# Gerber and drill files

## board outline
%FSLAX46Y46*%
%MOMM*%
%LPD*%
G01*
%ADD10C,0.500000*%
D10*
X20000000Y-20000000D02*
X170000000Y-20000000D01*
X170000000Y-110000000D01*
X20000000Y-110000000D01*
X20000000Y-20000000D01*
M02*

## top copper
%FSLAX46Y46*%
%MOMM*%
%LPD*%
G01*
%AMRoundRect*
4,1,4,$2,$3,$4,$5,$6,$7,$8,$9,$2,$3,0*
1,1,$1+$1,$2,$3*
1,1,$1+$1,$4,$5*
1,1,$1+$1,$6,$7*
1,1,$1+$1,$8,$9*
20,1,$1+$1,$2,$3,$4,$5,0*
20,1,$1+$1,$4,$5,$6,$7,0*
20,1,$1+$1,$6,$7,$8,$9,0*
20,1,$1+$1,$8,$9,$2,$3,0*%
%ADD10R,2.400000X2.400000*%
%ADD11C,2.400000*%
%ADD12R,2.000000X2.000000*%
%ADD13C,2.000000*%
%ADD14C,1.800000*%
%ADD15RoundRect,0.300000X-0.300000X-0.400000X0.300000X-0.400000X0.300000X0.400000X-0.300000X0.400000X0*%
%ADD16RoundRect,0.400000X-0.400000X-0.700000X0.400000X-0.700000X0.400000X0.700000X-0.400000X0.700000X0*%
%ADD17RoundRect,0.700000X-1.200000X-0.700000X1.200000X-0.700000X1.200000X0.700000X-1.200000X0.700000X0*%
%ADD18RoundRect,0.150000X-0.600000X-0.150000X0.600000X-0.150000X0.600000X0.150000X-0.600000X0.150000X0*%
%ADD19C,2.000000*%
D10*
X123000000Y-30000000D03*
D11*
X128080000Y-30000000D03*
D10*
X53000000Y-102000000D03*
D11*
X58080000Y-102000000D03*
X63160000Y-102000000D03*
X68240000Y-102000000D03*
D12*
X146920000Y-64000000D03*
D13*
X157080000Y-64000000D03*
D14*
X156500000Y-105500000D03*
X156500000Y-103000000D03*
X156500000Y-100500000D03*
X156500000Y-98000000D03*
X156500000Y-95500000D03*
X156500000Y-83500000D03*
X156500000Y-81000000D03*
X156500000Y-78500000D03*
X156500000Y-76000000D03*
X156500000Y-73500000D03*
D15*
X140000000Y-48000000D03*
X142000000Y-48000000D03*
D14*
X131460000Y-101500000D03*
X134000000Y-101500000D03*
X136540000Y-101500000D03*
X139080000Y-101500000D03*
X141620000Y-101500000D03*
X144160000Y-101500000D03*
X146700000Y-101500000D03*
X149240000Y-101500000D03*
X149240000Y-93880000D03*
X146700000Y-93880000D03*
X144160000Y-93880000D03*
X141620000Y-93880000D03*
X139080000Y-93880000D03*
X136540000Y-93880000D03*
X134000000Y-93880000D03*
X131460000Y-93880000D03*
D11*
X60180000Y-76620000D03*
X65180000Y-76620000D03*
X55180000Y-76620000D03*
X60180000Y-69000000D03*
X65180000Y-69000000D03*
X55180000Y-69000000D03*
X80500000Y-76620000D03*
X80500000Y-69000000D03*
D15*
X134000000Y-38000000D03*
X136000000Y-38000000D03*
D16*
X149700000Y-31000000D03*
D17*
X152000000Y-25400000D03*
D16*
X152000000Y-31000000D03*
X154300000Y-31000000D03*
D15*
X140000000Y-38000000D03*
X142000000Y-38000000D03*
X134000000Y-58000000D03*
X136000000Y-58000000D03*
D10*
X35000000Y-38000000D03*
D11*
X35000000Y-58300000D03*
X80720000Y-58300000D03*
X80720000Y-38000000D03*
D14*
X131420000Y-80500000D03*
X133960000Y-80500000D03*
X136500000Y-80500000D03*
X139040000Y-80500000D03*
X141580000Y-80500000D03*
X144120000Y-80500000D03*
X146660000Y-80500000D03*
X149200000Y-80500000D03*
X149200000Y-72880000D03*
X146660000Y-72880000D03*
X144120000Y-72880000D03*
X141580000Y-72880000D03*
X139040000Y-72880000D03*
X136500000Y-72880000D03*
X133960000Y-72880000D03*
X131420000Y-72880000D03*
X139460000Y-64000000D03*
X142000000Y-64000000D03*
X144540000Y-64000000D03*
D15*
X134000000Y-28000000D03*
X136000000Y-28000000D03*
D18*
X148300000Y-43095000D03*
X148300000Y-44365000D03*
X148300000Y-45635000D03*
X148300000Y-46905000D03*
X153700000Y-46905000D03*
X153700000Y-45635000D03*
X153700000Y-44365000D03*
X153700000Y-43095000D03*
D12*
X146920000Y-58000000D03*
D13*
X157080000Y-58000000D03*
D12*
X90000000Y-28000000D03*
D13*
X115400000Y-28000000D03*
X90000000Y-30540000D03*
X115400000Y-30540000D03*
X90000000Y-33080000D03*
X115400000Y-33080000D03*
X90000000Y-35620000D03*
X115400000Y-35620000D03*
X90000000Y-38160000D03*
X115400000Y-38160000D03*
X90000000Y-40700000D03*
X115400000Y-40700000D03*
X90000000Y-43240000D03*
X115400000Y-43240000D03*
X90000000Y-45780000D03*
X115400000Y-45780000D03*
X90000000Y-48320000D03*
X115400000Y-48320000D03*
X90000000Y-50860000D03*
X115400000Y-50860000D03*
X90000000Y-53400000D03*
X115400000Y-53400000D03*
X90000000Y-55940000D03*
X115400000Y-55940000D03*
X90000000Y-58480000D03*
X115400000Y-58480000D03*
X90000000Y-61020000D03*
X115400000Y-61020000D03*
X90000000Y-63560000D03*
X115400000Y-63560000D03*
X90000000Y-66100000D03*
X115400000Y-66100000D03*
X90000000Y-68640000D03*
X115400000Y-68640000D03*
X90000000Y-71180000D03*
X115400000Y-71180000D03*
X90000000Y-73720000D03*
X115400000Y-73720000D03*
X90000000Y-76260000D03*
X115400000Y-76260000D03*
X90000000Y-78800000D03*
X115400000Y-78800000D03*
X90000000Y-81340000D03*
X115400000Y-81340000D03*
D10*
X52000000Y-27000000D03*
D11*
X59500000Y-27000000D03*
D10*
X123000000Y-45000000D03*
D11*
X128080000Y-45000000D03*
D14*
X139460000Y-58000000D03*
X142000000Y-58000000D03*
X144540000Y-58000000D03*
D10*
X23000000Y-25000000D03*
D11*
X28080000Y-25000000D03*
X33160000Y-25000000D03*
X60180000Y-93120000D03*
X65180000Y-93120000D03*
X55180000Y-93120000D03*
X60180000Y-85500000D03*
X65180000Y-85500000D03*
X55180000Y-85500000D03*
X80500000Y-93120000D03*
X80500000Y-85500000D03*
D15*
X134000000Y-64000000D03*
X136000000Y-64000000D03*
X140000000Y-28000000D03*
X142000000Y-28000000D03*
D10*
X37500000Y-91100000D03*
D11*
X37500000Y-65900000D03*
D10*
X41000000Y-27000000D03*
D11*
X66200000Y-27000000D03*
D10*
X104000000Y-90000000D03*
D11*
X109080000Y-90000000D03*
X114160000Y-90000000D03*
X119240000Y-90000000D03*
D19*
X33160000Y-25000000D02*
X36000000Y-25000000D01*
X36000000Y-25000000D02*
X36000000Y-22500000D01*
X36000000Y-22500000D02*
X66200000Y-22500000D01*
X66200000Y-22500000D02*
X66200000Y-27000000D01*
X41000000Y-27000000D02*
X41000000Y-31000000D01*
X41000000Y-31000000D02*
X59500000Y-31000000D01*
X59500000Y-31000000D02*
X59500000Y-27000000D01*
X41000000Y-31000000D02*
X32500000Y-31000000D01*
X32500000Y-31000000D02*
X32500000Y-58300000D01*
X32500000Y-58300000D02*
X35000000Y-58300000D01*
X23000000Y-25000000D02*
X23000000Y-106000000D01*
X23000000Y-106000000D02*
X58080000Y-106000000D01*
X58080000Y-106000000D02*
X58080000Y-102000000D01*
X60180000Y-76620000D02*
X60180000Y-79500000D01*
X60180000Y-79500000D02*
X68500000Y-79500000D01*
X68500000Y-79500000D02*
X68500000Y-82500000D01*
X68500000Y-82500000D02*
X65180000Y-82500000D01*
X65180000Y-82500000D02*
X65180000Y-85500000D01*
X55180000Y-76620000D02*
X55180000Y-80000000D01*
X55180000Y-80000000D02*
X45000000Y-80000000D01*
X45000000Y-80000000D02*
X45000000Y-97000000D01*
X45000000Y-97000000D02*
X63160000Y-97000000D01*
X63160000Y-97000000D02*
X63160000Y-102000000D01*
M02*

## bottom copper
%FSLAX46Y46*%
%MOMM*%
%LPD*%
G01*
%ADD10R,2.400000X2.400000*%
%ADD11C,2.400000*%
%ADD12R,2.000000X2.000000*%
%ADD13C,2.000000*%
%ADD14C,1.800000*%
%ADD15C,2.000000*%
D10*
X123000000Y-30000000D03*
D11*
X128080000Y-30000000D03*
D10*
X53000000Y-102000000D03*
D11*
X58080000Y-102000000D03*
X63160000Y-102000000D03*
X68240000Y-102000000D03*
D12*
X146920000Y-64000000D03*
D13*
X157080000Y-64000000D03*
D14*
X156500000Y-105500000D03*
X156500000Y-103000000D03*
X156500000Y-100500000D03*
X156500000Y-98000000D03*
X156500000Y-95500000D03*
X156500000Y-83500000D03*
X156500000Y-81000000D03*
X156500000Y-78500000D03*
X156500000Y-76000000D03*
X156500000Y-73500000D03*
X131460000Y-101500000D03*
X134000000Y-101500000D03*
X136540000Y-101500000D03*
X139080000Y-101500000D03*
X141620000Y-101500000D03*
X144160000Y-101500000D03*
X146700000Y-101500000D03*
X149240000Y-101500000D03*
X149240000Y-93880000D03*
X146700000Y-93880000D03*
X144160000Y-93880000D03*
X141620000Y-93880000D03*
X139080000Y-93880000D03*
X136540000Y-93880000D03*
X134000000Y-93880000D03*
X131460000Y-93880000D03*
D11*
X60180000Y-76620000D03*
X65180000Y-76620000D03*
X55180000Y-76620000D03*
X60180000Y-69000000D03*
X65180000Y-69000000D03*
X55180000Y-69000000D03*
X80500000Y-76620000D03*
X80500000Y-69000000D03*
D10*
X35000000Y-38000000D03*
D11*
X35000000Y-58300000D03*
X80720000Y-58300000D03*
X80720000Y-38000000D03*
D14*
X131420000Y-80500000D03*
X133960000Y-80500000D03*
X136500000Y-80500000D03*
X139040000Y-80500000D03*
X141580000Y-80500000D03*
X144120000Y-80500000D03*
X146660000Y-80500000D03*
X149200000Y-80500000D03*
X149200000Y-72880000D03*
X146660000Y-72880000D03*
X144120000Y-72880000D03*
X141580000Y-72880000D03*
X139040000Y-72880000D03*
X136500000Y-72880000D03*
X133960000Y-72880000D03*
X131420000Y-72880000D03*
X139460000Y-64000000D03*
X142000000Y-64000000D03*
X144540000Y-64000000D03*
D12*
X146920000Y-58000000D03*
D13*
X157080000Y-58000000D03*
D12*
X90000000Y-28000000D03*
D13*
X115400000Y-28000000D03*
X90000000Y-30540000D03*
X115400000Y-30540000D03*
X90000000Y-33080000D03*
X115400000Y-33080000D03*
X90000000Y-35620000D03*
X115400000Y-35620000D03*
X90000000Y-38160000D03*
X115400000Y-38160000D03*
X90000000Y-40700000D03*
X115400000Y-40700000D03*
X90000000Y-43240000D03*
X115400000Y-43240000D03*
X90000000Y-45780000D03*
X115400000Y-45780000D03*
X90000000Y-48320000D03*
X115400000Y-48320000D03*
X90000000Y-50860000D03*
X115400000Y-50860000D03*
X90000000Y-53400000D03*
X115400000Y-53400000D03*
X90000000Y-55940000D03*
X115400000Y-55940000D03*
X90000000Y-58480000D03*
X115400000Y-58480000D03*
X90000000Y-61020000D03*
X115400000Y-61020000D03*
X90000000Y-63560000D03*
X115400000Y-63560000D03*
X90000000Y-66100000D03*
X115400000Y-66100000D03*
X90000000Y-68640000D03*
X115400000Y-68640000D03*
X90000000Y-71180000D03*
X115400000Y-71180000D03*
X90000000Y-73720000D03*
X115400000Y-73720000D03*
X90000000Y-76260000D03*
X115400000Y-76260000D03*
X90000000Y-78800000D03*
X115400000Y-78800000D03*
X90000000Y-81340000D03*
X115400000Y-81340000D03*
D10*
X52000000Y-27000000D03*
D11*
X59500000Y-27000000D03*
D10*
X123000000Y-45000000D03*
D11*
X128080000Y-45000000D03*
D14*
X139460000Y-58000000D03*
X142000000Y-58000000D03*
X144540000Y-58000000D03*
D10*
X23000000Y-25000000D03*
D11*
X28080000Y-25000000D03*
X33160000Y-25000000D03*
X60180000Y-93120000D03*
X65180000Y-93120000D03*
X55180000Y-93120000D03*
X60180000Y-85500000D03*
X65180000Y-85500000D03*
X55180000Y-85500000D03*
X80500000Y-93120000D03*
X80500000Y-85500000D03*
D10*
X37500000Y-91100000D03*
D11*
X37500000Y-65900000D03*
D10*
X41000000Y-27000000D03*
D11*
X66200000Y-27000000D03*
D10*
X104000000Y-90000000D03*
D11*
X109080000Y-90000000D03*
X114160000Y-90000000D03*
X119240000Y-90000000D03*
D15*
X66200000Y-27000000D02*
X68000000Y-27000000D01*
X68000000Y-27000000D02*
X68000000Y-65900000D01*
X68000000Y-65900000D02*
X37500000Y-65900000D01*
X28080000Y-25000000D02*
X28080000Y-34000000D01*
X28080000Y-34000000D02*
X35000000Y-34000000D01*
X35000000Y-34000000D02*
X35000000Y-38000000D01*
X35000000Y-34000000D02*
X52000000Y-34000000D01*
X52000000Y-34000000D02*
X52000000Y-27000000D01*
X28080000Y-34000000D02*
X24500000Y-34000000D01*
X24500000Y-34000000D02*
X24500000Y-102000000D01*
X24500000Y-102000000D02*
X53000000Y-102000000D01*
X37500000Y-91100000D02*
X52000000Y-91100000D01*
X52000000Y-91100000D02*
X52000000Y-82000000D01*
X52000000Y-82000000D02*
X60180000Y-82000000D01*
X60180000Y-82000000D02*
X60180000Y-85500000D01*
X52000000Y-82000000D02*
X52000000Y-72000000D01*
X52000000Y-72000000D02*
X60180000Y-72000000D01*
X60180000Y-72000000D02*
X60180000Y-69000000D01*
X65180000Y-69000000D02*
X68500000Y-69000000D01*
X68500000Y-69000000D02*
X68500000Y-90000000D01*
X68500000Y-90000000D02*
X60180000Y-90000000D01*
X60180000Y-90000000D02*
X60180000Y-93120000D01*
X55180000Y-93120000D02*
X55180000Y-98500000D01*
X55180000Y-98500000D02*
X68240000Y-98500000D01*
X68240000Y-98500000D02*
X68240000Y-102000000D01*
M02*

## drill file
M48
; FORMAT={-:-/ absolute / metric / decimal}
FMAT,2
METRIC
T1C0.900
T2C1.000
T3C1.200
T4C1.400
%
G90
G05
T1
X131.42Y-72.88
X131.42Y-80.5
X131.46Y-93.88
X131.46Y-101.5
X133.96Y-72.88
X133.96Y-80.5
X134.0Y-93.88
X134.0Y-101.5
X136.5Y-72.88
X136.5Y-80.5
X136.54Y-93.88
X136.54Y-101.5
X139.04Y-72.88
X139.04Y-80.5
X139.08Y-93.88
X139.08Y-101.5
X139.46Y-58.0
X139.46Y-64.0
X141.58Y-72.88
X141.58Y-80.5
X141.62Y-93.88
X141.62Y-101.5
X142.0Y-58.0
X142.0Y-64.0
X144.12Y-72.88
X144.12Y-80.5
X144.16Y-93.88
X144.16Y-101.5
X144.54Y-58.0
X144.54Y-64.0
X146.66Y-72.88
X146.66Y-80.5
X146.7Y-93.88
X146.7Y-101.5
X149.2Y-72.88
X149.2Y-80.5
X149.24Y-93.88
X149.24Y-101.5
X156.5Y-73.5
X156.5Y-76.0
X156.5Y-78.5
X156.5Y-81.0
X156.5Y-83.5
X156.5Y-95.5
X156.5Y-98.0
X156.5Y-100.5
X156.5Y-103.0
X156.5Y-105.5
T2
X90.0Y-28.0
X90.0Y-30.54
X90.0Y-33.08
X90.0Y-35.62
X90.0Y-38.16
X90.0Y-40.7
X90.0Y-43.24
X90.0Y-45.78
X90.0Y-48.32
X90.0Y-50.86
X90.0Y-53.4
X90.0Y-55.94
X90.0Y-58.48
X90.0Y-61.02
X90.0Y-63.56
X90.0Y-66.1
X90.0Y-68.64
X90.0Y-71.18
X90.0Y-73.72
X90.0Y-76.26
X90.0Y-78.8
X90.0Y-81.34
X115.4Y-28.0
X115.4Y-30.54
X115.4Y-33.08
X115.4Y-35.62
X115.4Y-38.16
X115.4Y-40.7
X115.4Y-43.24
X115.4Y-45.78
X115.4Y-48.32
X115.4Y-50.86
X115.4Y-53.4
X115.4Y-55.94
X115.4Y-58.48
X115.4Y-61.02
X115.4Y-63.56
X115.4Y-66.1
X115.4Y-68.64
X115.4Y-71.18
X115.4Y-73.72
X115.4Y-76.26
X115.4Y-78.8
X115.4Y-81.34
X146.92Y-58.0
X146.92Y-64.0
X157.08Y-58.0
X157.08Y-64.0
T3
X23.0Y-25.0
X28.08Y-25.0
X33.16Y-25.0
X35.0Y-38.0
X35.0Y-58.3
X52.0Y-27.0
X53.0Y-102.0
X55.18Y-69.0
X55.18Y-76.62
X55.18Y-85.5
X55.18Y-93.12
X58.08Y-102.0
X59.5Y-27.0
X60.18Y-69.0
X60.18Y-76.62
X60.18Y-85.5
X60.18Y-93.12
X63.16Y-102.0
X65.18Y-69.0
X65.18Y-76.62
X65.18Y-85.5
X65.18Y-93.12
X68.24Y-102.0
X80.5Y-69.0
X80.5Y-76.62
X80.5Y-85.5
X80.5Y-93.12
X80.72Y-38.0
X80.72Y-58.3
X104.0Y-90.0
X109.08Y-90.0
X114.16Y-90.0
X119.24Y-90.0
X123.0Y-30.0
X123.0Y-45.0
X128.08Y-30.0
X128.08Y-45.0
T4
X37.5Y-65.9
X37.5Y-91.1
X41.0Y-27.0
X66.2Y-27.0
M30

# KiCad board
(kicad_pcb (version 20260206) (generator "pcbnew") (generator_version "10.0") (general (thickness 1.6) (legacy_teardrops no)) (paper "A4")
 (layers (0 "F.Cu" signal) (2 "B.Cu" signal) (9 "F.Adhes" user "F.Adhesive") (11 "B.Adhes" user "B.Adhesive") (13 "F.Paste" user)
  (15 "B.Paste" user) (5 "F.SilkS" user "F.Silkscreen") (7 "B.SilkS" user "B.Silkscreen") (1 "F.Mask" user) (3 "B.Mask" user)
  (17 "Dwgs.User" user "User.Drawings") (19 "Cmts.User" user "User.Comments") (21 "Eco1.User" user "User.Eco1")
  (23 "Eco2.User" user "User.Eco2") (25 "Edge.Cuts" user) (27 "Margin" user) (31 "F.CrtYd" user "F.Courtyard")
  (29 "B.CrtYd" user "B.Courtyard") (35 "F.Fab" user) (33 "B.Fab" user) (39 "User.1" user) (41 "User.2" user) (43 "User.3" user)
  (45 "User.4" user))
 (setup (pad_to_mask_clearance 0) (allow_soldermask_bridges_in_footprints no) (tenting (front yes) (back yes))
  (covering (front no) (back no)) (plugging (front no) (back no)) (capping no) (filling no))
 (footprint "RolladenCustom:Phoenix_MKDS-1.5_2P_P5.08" (layer "F.Cu") (at 123 30)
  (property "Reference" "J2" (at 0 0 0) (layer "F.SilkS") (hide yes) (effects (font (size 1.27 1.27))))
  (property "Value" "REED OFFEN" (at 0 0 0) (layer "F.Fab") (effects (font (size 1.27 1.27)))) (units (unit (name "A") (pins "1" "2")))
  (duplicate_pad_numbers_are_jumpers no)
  (pad "1" thru_hole rect (at 0 0) (size 2.4 2.4) (drill 1.2) (layers "*.Cu" "*.Mask") (remove_unused_layers no) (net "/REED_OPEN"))
  (pad "2" thru_hole circle (at 5.08 0) (size 2.4 2.4) (drill 1.2) (layers "*.Cu" "*.Mask") (remove_unused_layers no) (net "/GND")))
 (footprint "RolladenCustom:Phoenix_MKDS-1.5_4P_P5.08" (layer "F.Cu") (at 53 102)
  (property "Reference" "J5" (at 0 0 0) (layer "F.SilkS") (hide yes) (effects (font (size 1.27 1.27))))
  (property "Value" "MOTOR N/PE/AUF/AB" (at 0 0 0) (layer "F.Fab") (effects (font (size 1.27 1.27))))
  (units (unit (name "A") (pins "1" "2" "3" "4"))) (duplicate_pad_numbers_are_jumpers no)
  (pad "1" thru_hole rect (at 0 0) (size 2.4 2.4) (drill 1.2) (layers "*.Cu" "*.Mask") (remove_unused_layers no) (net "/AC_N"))
  (pad "2" thru_hole circle (at 5.08 0) (size 2.4 2.4) (drill 1.2) (layers "*.Cu" "*.Mask") (remove_unused_layers no) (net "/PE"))
  (pad "3" thru_hole circle (at 10.16 0) (size 2.4 2.4) (drill 1.2) (layers "*.Cu" "*.Mask") (remove_unused_layers no) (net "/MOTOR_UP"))
  (pad "4" thru_hole circle (at 15.24 0) (size 2.4 2.4) (drill 1.2) (layers "*.Cu" "*.Mask") (remove_unused_layers no) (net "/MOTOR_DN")))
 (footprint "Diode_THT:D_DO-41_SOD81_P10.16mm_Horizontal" (layer "F.Cu") (at 152 64)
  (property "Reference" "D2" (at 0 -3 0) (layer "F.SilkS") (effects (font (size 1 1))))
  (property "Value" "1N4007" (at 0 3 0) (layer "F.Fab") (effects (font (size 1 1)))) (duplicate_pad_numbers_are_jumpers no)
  (pad "1" thru_hole rect (at -5.08 0) (size 2 2) (drill 1) (layers "*.Cu" "*.Mask") (remove_unused_layers no) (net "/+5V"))
  (pad "2" thru_hole circle (at 5.08 0) (size 2 2) (drill 1) (layers "*.Cu" "*.Mask") (remove_unused_layers no) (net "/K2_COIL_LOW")))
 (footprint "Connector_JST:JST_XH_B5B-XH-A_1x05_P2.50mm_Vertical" (layer "F.Cu") (at 156.5 105.5 90)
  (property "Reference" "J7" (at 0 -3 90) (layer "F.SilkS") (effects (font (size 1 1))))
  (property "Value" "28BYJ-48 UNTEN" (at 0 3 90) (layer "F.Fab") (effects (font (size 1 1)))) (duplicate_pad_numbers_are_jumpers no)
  (pad "1" thru_hole circle (at 0 0 90) (size 1.8 1.8) (drill 0.9) (layers "*.Cu" "*.Mask") (remove_unused_layers no) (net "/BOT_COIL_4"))
  (pad "2" thru_hole circle (at 2.5 0 90) (size 1.8 1.8) (drill 0.9) (layers "*.Cu" "*.Mask") (remove_unused_layers no) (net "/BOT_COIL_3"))
  (pad "3" thru_hole circle (at 5 0 90) (size 1.8 1.8) (drill 0.9) (layers "*.Cu" "*.Mask") (remove_unused_layers no) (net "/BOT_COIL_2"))
  (pad "4" thru_hole circle (at 7.5 0 90) (size 1.8 1.8) (drill 0.9) (layers "*.Cu" "*.Mask") (remove_unused_layers no) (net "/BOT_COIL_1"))
  (pad "5" thru_hole circle (at 10 0 90) (size 1.8 1.8) (drill 0.9) (layers "*.Cu" "*.Mask") (remove_unused_layers no) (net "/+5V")))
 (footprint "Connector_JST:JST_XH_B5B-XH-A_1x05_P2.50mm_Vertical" (layer "F.Cu") (at 156.5 83.5 90)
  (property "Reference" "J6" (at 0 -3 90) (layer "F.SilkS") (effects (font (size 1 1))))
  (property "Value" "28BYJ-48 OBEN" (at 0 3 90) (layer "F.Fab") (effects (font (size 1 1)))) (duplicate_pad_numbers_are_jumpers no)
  (pad "1" thru_hole circle (at 0 0 90) (size 1.8 1.8) (drill 0.9) (layers "*.Cu" "*.Mask") (remove_unused_layers no) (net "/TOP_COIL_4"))
  (pad "2" thru_hole circle (at 2.5 0 90) (size 1.8 1.8) (drill 0.9) (layers "*.Cu" "*.Mask") (remove_unused_layers no) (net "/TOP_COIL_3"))
  (pad "3" thru_hole circle (at 5 0 90) (size 1.8 1.8) (drill 0.9) (layers "*.Cu" "*.Mask") (remove_unused_layers no) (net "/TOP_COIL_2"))
  (pad "4" thru_hole circle (at 7.5 0 90) (size 1.8 1.8) (drill 0.9) (layers "*.Cu" "*.Mask") (remove_unused_layers no) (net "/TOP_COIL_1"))
  (pad "5" thru_hole circle (at 10 0 90) (size 1.8 1.8) (drill 0.9) (layers "*.Cu" "*.Mask") (remove_unused_layers no) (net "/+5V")))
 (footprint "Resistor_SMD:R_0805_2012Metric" (layer "F.Cu") (at 141 48)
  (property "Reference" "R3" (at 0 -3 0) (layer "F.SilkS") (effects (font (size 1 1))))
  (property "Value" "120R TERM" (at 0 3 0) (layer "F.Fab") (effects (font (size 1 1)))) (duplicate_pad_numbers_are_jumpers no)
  (pad "1" smd roundrect (at -1 0) (size 1.2 1.4) (layers "F.Cu" "F.Mask" "F.Paste") (roundrect_rratio 0.25) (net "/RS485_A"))
  (pad "2" smd roundrect (at 1 0) (size 1.2 1.4) (layers "F.Cu" "F.Mask" "F.Paste") (roundrect_rratio 0.25) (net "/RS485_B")))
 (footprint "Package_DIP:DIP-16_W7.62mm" (layer "F.Cu") (at 131.46 101.5 90)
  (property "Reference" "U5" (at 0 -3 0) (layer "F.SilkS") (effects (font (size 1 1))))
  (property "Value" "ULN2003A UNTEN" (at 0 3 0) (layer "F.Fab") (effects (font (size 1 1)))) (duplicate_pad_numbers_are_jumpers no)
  (pad "1" thru_hole circle (at 0 0) (size 1.8 1.8) (drill 0.9) (layers "*.Cu" "*.Mask") (remove_unused_layers no) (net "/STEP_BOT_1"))
  (pad "2" thru_hole circle (at 0 2.54) (size 1.8 1.8) (drill 0.9) (layers "*.Cu" "*.Mask") (remove_unused_layers no) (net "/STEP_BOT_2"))
  (pad "3" thru_hole circle (at 0 5.08) (size 1.8 1.8) (drill 0.9) (layers "*.Cu" "*.Mask") (remove_unused_layers no) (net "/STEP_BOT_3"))
  (pad "4" thru_hole circle (at 0 7.62) (size 1.8 1.8) (drill 0.9) (layers "*.Cu" "*.Mask") (remove_unused_layers no) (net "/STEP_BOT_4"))
  (pad "5" thru_hole circle (at 0 10.16) (size 1.8 1.8) (drill 0.9) (layers "*.Cu" "*.Mask") (remove_unused_layers no))
  (pad "6" thru_hole circle (at 0 12.7) (size 1.8 1.8) (drill 0.9) (layers "*.Cu" "*.Mask") (remove_unused_layers no))
  (pad "7" thru_hole circle (at 0 15.24) (size 1.8 1.8) (drill 0.9) (layers "*.Cu" "*.Mask") (remove_unused_layers no))
  (pad "8" thru_hole circle (at 0 17.78) (size 1.8 1.8) (drill 0.9) (layers "*.Cu" "*.Mask") (remove_unused_layers no) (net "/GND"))
  (pad "9" thru_hole circle (at 7.62 17.78) (size 1.8 1.8) (drill 0.9) (layers "*.Cu" "*.Mask") (remove_unused_layers no) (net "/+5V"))
  (pad "10" thru_hole circle (at 7.62 15.24) (size 1.8 1.8) (drill 0.9) (layers "*.Cu" "*.Mask") (remove_unused_layers no))
  (pad "11" thru_hole circle (at 7.62 12.7) (size 1.8 1.8) (drill 0.9) (layers "*.Cu" "*.Mask") (remove_unused_layers no))
  (pad "12" thru_hole circle (at 7.62 10.16) (size 1.8 1.8) (drill 0.9) (layers "*.Cu" "*.Mask") (remove_unused_layers no))
  (pad "13" thru_hole circle (at 7.62 7.62) (size 1.8 1.8) (drill 0.9) (layers "*.Cu" "*.Mask") (remove_unused_layers no)
   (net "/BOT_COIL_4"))
  (pad "14" thru_hole circle (at 7.62 5.08) (size 1.8 1.8) (drill 0.9) (layers "*.Cu" "*.Mask") (remove_unused_layers no)
   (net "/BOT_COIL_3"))
  (pad "15" thru_hole circle (at 7.62 2.54) (size 1.8 1.8) (drill 0.9) (layers "*.Cu" "*.Mask") (remove_unused_layers no)
   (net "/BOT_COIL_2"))
  (pad "16" thru_hole circle (at 7.62 0) (size 1.8 1.8) (drill 0.9) (layers "*.Cu" "*.Mask") (remove_unused_layers no) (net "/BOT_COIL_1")))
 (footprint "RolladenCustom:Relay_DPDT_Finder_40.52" (layer "F.Cu") (at 80.5 76.62 180)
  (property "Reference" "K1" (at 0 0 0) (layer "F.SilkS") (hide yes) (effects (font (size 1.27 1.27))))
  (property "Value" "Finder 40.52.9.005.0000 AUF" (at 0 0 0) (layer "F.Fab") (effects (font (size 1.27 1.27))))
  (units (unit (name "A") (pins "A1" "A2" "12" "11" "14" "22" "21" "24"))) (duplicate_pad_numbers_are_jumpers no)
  (pad "11" thru_hole circle (at 20.32 0) (size 2.4 2.4) (drill 1.2) (layers "*.Cu" "*.Mask") (remove_unused_layers no) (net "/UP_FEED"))
  (pad "12" thru_hole circle (at 15.32 0) (size 2.4 2.4) (drill 1.2) (layers "*.Cu" "*.Mask") (remove_unused_layers no)
   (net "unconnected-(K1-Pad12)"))
  (pad "14" thru_hole circle (at 25.32 0) (size 2.4 2.4) (drill 1.2) (layers "*.Cu" "*.Mask") (remove_unused_layers no) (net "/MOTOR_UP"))
  (pad "21" thru_hole circle (at 20.32 7.62) (size 2.4 2.4) (drill 1.2) (layers "*.Cu" "*.Mask") (remove_unused_layers no) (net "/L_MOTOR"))
  (pad "22" thru_hole circle (at 15.32 7.62) (size 2.4 2.4) (drill 1.2) (layers "*.Cu" "*.Mask") (remove_unused_layers no) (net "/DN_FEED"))
  (pad "24" thru_hole circle (at 25.32 7.62) (size 2.4 2.4) (drill 1.2) (layers "*.Cu" "*.Mask") (remove_unused_layers no)
   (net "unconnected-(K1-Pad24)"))
  (pad "A1" thru_hole circle (at 0 0) (size 2.4 2.4) (drill 1.2) (layers "*.Cu" "*.Mask") (remove_unused_layers no) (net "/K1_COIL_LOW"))
  (pad "A2" thru_hole circle (at 0 7.62) (size 2.4 2.4) (drill 1.2) (layers "*.Cu" "*.Mask") (remove_unused_layers no) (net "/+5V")))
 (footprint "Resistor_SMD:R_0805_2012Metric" (layer "F.Cu") (at 135 38)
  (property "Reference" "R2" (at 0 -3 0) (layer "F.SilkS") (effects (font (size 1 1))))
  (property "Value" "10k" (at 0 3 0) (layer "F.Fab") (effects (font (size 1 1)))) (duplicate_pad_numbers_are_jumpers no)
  (pad "1" smd roundrect (at -1 0) (size 1.2 1.4) (layers "F.Cu" "F.Mask" "F.Paste") (roundrect_rratio 0.25) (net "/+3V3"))
  (pad "2" smd roundrect (at 1 0) (size 1.2 1.4) (layers "F.Cu" "F.Mask" "F.Paste") (roundrect_rratio 0.25) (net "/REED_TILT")))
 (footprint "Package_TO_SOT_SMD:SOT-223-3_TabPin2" (layer "F.Cu") (at 152 28)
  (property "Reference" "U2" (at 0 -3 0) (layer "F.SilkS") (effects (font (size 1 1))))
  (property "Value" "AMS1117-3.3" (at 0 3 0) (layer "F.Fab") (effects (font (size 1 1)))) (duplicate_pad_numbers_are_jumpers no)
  (pad "1" smd roundrect (at -2.3 3) (size 1.6 2.2) (layers "F.Cu" "F.Mask" "F.Paste") (roundrect_rratio 0.25) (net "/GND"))
  (pad "2" smd roundrect (at 0 -2.6) (size 3.8 2.8) (layers "F.Cu" "F.Mask" "F.Paste") (roundrect_rratio 0.25) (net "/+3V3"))
  (pad "2" smd roundrect (at 0 3) (size 1.6 2.2) (layers "F.Cu" "F.Mask" "F.Paste") (roundrect_rratio 0.25) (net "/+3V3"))
  (pad "3" smd roundrect (at 2.3 3) (size 1.6 2.2) (layers "F.Cu" "F.Mask" "F.Paste") (roundrect_rratio 0.25) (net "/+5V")))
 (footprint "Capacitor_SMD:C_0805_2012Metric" (layer "F.Cu") (at 141 38)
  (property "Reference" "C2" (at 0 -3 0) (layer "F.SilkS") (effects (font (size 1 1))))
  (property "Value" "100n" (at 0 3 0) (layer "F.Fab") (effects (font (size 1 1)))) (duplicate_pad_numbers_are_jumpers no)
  (pad "1" smd roundrect (at -1 0) (size 1.2 1.4) (layers "F.Cu" "F.Mask" "F.Paste") (roundrect_rratio 0.25) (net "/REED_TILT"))
  (pad "2" smd roundrect (at 1 0) (size 1.2 1.4) (layers "F.Cu" "F.Mask" "F.Paste") (roundrect_rratio 0.25) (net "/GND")))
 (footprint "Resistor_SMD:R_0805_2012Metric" (layer "F.Cu") (at 135 58)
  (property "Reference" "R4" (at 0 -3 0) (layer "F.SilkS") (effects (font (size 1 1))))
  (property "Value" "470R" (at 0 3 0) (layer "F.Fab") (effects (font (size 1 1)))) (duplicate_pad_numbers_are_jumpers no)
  (pad "1" smd roundrect (at -1 0) (size 1.2 1.4) (layers "F.Cu" "F.Mask" "F.Paste") (roundrect_rratio 0.25) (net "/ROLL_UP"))
  (pad "2" smd roundrect (at 1 0) (size 1.2 1.4) (layers "F.Cu" "F.Mask" "F.Paste") (roundrect_rratio 0.25) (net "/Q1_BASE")))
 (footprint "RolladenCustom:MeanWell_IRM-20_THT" (layer "F.Cu") (at 35 38)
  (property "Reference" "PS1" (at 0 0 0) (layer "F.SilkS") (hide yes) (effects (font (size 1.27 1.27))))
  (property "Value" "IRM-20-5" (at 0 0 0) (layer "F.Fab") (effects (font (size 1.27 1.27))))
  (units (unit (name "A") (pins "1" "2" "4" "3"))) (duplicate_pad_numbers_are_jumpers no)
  (pad "1" thru_hole rect (at 0 0) (size 2.4 2.4) (drill 1.2) (layers "*.Cu" "*.Mask") (remove_unused_layers no) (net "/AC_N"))
  (pad "2" thru_hole circle (at 0 20.3) (size 2.4 2.4) (drill 1.2) (layers "*.Cu" "*.Mask") (remove_unused_layers no) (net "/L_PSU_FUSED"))
  (pad "3" thru_hole circle (at 45.72 20.3) (size 2.4 2.4) (drill 1.2) (layers "*.Cu" "*.Mask") (remove_unused_layers no) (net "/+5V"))
  (pad "4" thru_hole circle (at 45.72 0) (size 2.4 2.4) (drill 1.2) (layers "*.Cu" "*.Mask") (remove_unused_layers no) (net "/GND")))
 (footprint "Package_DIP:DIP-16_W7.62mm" (layer "F.Cu") (at 131.42 80.5 90)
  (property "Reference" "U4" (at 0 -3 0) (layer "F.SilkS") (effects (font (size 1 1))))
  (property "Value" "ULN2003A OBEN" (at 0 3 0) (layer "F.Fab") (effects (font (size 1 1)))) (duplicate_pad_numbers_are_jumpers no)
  (pad "1" thru_hole circle (at 0 0) (size 1.8 1.8) (drill 0.9) (layers "*.Cu" "*.Mask") (remove_unused_layers no) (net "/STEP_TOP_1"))
  (pad "2" thru_hole circle (at 0 2.54) (size 1.8 1.8) (drill 0.9) (layers "*.Cu" "*.Mask") (remove_unused_layers no) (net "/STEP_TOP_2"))
  (pad "3" thru_hole circle (at 0 5.08) (size 1.8 1.8) (drill 0.9) (layers "*.Cu" "*.Mask") (remove_unused_layers no) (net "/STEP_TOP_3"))
  (pad "4" thru_hole circle (at 0 7.62) (size 1.8 1.8) (drill 0.9) (layers "*.Cu" "*.Mask") (remove_unused_layers no) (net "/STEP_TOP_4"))
  (pad "5" thru_hole circle (at 0 10.16) (size 1.8 1.8) (drill 0.9) (layers "*.Cu" "*.Mask") (remove_unused_layers no))
  (pad "6" thru_hole circle (at 0 12.7) (size 1.8 1.8) (drill 0.9) (layers "*.Cu" "*.Mask") (remove_unused_layers no))
  (pad "7" thru_hole circle (at 0 15.24) (size 1.8 1.8) (drill 0.9) (layers "*.Cu" "*.Mask") (remove_unused_layers no))
  (pad "8" thru_hole circle (at 0 17.78) (size 1.8 1.8) (drill 0.9) (layers "*.Cu" "*.Mask") (remove_unused_layers no) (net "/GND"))
  (pad "9" thru_hole circle (at 7.62 17.78) (size 1.8 1.8) (drill 0.9) (layers "*.Cu" "*.Mask") (remove_unused_layers no) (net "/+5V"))
  (pad "10" thru_hole circle (at 7.62 15.24) (size 1.8 1.8) (drill 0.9) (layers "*.Cu" "*.Mask") (remove_unused_layers no))
  (pad "11" thru_hole circle (at 7.62 12.7) (size 1.8 1.8) (drill 0.9) (layers "*.Cu" "*.Mask") (remove_unused_layers no))
  (pad "12" thru_hole circle (at 7.62 10.16) (size 1.8 1.8) (drill 0.9) (layers "*.Cu" "*.Mask") (remove_unused_layers no))
  (pad "13" thru_hole circle (at 7.62 7.62) (size 1.8 1.8) (drill 0.9) (layers "*.Cu" "*.Mask") (remove_unused_layers no)
   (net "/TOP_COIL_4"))
  (pad "14" thru_hole circle (at 7.62 5.08) (size 1.8 1.8) (drill 0.9) (layers "*.Cu" "*.Mask") (remove_unused_layers no)
   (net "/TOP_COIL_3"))
  (pad "15" thru_hole circle (at 7.62 2.54) (size 1.8 1.8) (drill 0.9) (layers "*.Cu" "*.Mask") (remove_unused_layers no)
   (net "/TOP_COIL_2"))
  (pad "16" thru_hole circle (at 7.62 0) (size 1.8 1.8) (drill 0.9) (layers "*.Cu" "*.Mask") (remove_unused_layers no) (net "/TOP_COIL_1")))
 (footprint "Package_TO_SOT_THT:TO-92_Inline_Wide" (layer "F.Cu") (at 142 64)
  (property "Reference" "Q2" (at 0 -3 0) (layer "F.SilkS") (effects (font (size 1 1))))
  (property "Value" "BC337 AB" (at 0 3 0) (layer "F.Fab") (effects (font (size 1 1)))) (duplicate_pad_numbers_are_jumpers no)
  (pad "1" thru_hole circle (at -2.54 0) (size 1.8 1.8) (drill 0.9) (layers "*.Cu" "*.Mask") (remove_unused_layers no) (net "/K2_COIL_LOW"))
  (pad "2" thru_hole circle (at 0 0) (size 1.8 1.8) (drill 0.9) (layers "*.Cu" "*.Mask") (remove_unused_layers no) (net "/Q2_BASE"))
  (pad "3" thru_hole circle (at 2.54 0) (size 1.8 1.8) (drill 0.9) (layers "*.Cu" "*.Mask") (remove_unused_layers no) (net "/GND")))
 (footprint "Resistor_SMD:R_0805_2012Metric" (layer "F.Cu") (at 135 28)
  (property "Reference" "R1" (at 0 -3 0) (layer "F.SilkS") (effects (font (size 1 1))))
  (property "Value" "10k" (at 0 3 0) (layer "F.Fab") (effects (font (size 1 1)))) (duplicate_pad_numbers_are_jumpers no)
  (pad "1" smd roundrect (at -1 0) (size 1.2 1.4) (layers "F.Cu" "F.Mask" "F.Paste") (roundrect_rratio 0.25) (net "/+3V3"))
  (pad "2" smd roundrect (at 1 0) (size 1.2 1.4) (layers "F.Cu" "F.Mask" "F.Paste") (roundrect_rratio 0.25) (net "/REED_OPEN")))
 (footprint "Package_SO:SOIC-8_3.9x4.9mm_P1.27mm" (layer "F.Cu") (at 151 45)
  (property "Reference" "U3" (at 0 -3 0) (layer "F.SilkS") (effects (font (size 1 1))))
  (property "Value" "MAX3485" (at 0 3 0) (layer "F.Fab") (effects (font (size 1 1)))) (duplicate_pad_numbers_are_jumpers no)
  (pad "1" smd roundrect (at -2.7 -1.905) (size 1.5 0.6) (layers "F.Cu" "F.Mask" "F.Paste") (roundrect_rratio 0.25) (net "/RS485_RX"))
  (pad "2" smd roundrect (at -2.7 -0.635) (size 1.5 0.6) (layers "F.Cu" "F.Mask" "F.Paste") (roundrect_rratio 0.25) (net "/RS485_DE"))
  (pad "3" smd roundrect (at -2.7 0.635) (size 1.5 0.6) (layers "F.Cu" "F.Mask" "F.Paste") (roundrect_rratio 0.25) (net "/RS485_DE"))
  (pad "4" smd roundrect (at -2.7 1.905) (size 1.5 0.6) (layers "F.Cu" "F.Mask" "F.Paste") (roundrect_rratio 0.25) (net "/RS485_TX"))
  (pad "5" smd roundrect (at 2.7 1.905) (size 1.5 0.6) (layers "F.Cu" "F.Mask" "F.Paste") (roundrect_rratio 0.25) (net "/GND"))
  (pad "6" smd roundrect (at 2.7 0.635) (size 1.5 0.6) (layers "F.Cu" "F.Mask" "F.Paste") (roundrect_rratio 0.25) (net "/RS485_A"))
  (pad "7" smd roundrect (at 2.7 -0.635) (size 1.5 0.6) (layers "F.Cu" "F.Mask" "F.Paste") (roundrect_rratio 0.25) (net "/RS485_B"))
  (pad "8" smd roundrect (at 2.7 -1.905) (size 1.5 0.6) (layers "F.Cu" "F.Mask" "F.Paste") (roundrect_rratio 0.25) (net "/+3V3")))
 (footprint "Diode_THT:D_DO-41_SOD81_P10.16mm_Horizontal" (layer "F.Cu") (at 152 58)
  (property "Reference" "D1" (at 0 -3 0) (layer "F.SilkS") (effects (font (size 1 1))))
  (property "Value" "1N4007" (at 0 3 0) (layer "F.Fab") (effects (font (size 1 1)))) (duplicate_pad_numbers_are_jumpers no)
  (pad "1" thru_hole rect (at -5.08 0) (size 2 2) (drill 1) (layers "*.Cu" "*.Mask") (remove_unused_layers no) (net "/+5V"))
  (pad "2" thru_hole circle (at 5.08 0) (size 2 2) (drill 1) (layers "*.Cu" "*.Mask") (remove_unused_layers no) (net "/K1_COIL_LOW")))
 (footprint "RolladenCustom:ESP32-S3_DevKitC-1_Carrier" (layer "F.Cu") (at 90 28)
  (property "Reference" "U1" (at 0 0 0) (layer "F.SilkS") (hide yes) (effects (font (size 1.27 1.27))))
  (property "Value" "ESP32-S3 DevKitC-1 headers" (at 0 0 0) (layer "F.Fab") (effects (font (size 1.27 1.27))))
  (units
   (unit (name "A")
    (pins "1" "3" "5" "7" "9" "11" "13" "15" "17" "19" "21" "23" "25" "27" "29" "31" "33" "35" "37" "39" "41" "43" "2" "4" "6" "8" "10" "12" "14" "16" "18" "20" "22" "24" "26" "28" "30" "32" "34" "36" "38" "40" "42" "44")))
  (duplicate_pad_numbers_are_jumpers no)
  (pad "1" thru_hole rect (at 0 0) (size 2 2) (drill 1) (layers "*.Cu" "*.Mask") (remove_unused_layers no) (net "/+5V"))
  (pad "2" thru_hole circle (at 25.4 0) (size 2 2) (drill 1) (layers "*.Cu" "*.Mask") (remove_unused_layers no) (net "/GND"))
  (pad "3" thru_hole circle (at 0 2.54) (size 2 2) (drill 1) (layers "*.Cu" "*.Mask") (remove_unused_layers no) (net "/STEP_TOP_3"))
  (pad "4" thru_hole circle (at 25.4 2.54) (size 2 2) (drill 1) (layers "*.Cu" "*.Mask") (remove_unused_layers no)
   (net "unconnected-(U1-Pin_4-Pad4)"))
  (pad "5" thru_hole circle (at 0 5.08) (size 2 2) (drill 1) (layers "*.Cu" "*.Mask") (remove_unused_layers no) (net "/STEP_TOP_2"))
  (pad "6" thru_hole circle (at 25.4 5.08) (size 2 2) (drill 1) (layers "*.Cu" "*.Mask") (remove_unused_layers no)
   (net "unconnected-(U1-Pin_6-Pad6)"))
  (pad "7" thru_hole circle (at 0 7.62) (size 2 2) (drill 1) (layers "*.Cu" "*.Mask") (remove_unused_layers no) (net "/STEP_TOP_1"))
  (pad "8" thru_hole circle (at 25.4 7.62) (size 2 2) (drill 1) (layers "*.Cu" "*.Mask") (remove_unused_layers no)
   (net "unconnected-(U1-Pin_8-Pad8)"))
  (pad "9" thru_hole circle (at 0 10.16) (size 2 2) (drill 1) (layers "*.Cu" "*.Mask") (remove_unused_layers no) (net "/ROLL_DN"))
  (pad "10" thru_hole circle (at 25.4 10.16) (size 2 2) (drill 1) (layers "*.Cu" "*.Mask") (remove_unused_layers no)
   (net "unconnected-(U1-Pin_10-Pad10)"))
  (pad "11" thru_hole circle (at 0 12.7) (size 2 2) (drill 1) (layers "*.Cu" "*.Mask") (remove_unused_layers no) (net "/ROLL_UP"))
  (pad "12" thru_hole circle (at 25.4 12.7) (size 2 2) (drill 1) (layers "*.Cu" "*.Mask") (remove_unused_layers no)
   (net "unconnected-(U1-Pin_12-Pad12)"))
  (pad "13" thru_hole circle (at 0 15.24) (size 2 2) (drill 1) (layers "*.Cu" "*.Mask") (remove_unused_layers no)
   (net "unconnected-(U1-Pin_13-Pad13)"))
  (pad "14" thru_hole circle (at 25.4 15.24) (size 2 2) (drill 1) (layers "*.Cu" "*.Mask") (remove_unused_layers no)
   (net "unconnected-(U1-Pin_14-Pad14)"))
  (pad "15" thru_hole circle (at 0 17.78) (size 2 2) (drill 1) (layers "*.Cu" "*.Mask") (remove_unused_layers no)
   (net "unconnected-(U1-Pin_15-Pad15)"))
  (pad "16" thru_hole circle (at 25.4 17.78) (size 2 2) (drill 1) (layers "*.Cu" "*.Mask") (remove_unused_layers no)
   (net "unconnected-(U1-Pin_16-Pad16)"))
  (pad "17" thru_hole circle (at 0 20.32) (size 2 2) (drill 1) (layers "*.Cu" "*.Mask") (remove_unused_layers no)
   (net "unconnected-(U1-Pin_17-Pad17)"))
  (pad "18" thru_hole circle (at 25.4 20.32) (size 2 2) (drill 1) (layers "*.Cu" "*.Mask") (remove_unused_layers no)
   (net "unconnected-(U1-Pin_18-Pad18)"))
  (pad "19" thru_hole circle (at 0 22.86) (size 2 2) (drill 1) (layers "*.Cu" "*.Mask") (remove_unused_layers no)
   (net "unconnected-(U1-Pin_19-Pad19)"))
  (pad "20" thru_hole circle (at 25.4 22.86) (size 2 2) (drill 1) (layers "*.Cu" "*.Mask") (remove_unused_layers no)
   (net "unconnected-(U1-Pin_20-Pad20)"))
  (pad "21" thru_hole circle (at 0 25.4) (size 2 2) (drill 1) (layers "*.Cu" "*.Mask") (remove_unused_layers no) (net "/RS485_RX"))
  (pad "22" thru_hole circle (at 25.4 25.4) (size 2 2) (drill 1) (layers "*.Cu" "*.Mask") (remove_unused_layers no)
   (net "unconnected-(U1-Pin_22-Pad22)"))
  (pad "23" thru_hole circle (at 0 27.94) (size 2 2) (drill 1) (layers "*.Cu" "*.Mask") (remove_unused_layers no) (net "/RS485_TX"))
  (pad "24" thru_hole circle (at 25.4 27.94) (size 2 2) (drill 1) (layers "*.Cu" "*.Mask") (remove_unused_layers no) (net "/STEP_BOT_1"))
  (pad "25" thru_hole circle (at 0 30.48) (size 2 2) (drill 1) (layers "*.Cu" "*.Mask") (remove_unused_layers no) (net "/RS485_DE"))
  (pad "26" thru_hole circle (at 25.4 30.48) (size 2 2) (drill 1) (layers "*.Cu" "*.Mask") (remove_unused_layers no) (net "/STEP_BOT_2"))
  (pad "27" thru_hole circle (at 0 33.02) (size 2 2) (drill 1) (layers "*.Cu" "*.Mask") (remove_unused_layers no) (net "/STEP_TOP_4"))
  (pad "28" thru_hole circle (at 25.4 33.02) (size 2 2) (drill 1) (layers "*.Cu" "*.Mask") (remove_unused_layers no) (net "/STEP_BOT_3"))
  (pad "29" thru_hole circle (at 0 35.56) (size 2 2) (drill 1) (layers "*.Cu" "*.Mask") (remove_unused_layers no)
   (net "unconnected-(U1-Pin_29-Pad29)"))
  (pad "30" thru_hole circle (at 25.4 35.56) (size 2 2) (drill 1) (layers "*.Cu" "*.Mask") (remove_unused_layers no) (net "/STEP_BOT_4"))
  (pad "31" thru_hole circle (at 0 38.1) (size 2 2) (drill 1) (layers "*.Cu" "*.Mask") (remove_unused_layers no)
   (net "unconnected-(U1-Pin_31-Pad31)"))
  (pad "32" thru_hole circle (at 25.4 38.1) (size 2 2) (drill 1) (layers "*.Cu" "*.Mask") (remove_unused_layers no)
   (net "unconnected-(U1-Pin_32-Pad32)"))
  (pad "33" thru_hole circle (at 0 40.64) (size 2 2) (drill 1) (layers "*.Cu" "*.Mask") (remove_unused_layers no) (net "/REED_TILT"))
  (pad "34" thru_hole circle (at 25.4 40.64) (size 2 2) (drill 1) (layers "*.Cu" "*.Mask") (remove_unused_layers no)
   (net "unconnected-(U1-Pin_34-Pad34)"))
  (pad "35" thru_hole circle (at 0 43.18) (size 2 2) (drill 1) (layers "*.Cu" "*.Mask") (remove_unused_layers no) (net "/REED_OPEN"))
  (pad "36" thru_hole circle (at 25.4 43.18) (size 2 2) (drill 1) (layers "*.Cu" "*.Mask") (remove_unused_layers no)
   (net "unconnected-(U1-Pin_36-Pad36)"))
  (pad "37" thru_hole circle (at 0 45.72) (size 2 2) (drill 1) (layers "*.Cu" "*.Mask") (remove_unused_layers no)
   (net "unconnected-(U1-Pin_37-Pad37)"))
  (pad "38" thru_hole circle (at 25.4 45.72) (size 2 2) (drill 1) (layers "*.Cu" "*.Mask") (remove_unused_layers no)
   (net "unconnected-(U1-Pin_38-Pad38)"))
  (pad "39" thru_hole circle (at 0 48.26) (size 2 2) (drill 1) (layers "*.Cu" "*.Mask") (remove_unused_layers no)
   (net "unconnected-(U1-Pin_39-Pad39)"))
  (pad "40" thru_hole circle (at 25.4 48.26) (size 2 2) (drill 1) (layers "*.Cu" "*.Mask") (remove_unused_layers no)
   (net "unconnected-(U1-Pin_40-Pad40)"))
  (pad "41" thru_hole circle (at 0 50.8) (size 2 2) (drill 1) (layers "*.Cu" "*.Mask") (remove_unused_layers no)
   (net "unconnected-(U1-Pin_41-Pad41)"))
  (pad "42" thru_hole circle (at 25.4 50.8) (size 2 2) (drill 1) (layers "*.Cu" "*.Mask") (remove_unused_layers no) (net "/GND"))
  (pad "43" thru_hole circle (at 0 53.34) (size 2 2) (drill 1) (layers "*.Cu" "*.Mask") (remove_unused_layers no)
   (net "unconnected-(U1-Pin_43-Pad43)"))
  (pad "44" thru_hole circle (at 25.4 53.34) (size 2 2) (drill 1) (layers "*.Cu" "*.Mask") (remove_unused_layers no)
   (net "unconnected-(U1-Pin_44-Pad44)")))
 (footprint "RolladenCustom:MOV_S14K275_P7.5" (layer "F.Cu") (at 52 27)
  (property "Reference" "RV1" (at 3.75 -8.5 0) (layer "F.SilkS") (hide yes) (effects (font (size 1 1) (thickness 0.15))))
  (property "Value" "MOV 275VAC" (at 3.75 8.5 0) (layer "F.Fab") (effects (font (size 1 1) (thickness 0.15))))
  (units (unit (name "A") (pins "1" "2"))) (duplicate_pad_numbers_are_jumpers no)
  (pad "1" thru_hole rect (at 0 0) (size 2.4 2.4) (drill 1.2) (layers "*.Cu" "*.Mask") (remove_unused_layers no) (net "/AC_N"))
  (pad "2" thru_hole circle (at 7.5 0) (size 2.4 2.4) (drill 1.2) (layers "*.Cu" "*.Mask") (remove_unused_layers no) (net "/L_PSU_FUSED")))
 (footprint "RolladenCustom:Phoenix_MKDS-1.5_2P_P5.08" (layer "F.Cu") (at 123 45)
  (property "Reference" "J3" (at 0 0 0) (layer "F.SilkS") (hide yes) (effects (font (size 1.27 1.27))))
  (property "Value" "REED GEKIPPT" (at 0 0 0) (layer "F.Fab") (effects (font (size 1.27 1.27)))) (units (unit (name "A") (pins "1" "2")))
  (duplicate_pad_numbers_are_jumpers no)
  (pad "1" thru_hole rect (at 0 0) (size 2.4 2.4) (drill 1.2) (layers "*.Cu" "*.Mask") (remove_unused_layers no) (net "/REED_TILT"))
  (pad "2" thru_hole circle (at 5.08 0) (size 2.4 2.4) (drill 1.2) (layers "*.Cu" "*.Mask") (remove_unused_layers no) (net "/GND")))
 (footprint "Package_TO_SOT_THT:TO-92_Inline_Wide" (layer "F.Cu") (at 142 58)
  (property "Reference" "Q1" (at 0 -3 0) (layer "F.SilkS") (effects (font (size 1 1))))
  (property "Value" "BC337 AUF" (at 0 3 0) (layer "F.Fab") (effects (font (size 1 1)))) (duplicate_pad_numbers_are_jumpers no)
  (pad "1" thru_hole circle (at -2.54 0) (size 1.8 1.8) (drill 0.9) (layers "*.Cu" "*.Mask") (remove_unused_layers no) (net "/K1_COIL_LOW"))
  (pad "2" thru_hole circle (at 0 0) (size 1.8 1.8) (drill 0.9) (layers "*.Cu" "*.Mask") (remove_unused_layers no) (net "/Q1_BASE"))
  (pad "3" thru_hole circle (at 2.54 0) (size 1.8 1.8) (drill 0.9) (layers "*.Cu" "*.Mask") (remove_unused_layers no) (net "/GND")))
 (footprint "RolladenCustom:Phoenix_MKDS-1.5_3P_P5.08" (layer "F.Cu") (at 23 25)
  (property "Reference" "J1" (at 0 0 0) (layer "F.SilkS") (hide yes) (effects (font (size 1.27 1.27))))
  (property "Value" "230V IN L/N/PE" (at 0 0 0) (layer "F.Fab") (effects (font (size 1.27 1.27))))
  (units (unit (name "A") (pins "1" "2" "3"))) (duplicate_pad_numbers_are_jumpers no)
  (pad "1" thru_hole rect (at 0 0) (size 2.4 2.4) (drill 1.2) (layers "*.Cu" "*.Mask") (remove_unused_layers no) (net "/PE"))
  (pad "2" thru_hole circle (at 5.08 0) (size 2.4 2.4) (drill 1.2) (layers "*.Cu" "*.Mask") (remove_unused_layers no) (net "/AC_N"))
  (pad "3" thru_hole circle (at 10.16 0) (size 2.4 2.4) (drill 1.2) (layers "*.Cu" "*.Mask") (remove_unused_layers no) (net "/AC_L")))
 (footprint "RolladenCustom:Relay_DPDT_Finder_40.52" (layer "F.Cu") (at 80.5 93.12 180)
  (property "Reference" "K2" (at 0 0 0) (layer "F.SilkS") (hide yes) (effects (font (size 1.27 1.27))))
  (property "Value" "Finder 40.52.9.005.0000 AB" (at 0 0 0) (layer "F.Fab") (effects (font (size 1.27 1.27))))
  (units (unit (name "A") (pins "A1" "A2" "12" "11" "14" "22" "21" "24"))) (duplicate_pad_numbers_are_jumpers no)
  (pad "11" thru_hole circle (at 20.32 0) (size 2.4 2.4) (drill 1.2) (layers "*.Cu" "*.Mask") (remove_unused_layers no) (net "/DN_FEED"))
  (pad "12" thru_hole circle (at 15.32 0) (size 2.4 2.4) (drill 1.2) (layers "*.Cu" "*.Mask") (remove_unused_layers no)
   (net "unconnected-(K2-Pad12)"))
  (pad "14" thru_hole circle (at 25.32 0) (size 2.4 2.4) (drill 1.2) (layers "*.Cu" "*.Mask") (remove_unused_layers no) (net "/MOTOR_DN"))
  (pad "21" thru_hole circle (at 20.32 7.62) (size 2.4 2.4) (drill 1.2) (layers "*.Cu" "*.Mask") (remove_unused_layers no) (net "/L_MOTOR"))
  (pad "22" thru_hole circle (at 15.32 7.62) (size 2.4 2.4) (drill 1.2) (layers "*.Cu" "*.Mask") (remove_unused_layers no) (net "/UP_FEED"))
  (pad "24" thru_hole circle (at 25.32 7.62) (size 2.4 2.4) (drill 1.2) (layers "*.Cu" "*.Mask") (remove_unused_layers no)
   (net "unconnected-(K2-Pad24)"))
  (pad "A1" thru_hole circle (at 0 0) (size 2.4 2.4) (drill 1.2) (layers "*.Cu" "*.Mask") (remove_unused_layers no) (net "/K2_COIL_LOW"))
  (pad "A2" thru_hole circle (at 0 7.62) (size 2.4 2.4) (drill 1.2) (layers "*.Cu" "*.Mask") (remove_unused_layers no) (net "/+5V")))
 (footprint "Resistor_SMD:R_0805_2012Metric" (layer "F.Cu") (at 135 64)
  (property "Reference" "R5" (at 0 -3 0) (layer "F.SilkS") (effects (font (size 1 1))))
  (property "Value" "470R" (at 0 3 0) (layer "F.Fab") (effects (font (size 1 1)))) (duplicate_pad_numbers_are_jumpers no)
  (pad "1" smd roundrect (at -1 0) (size 1.2 1.4) (layers "F.Cu" "F.Mask" "F.Paste") (roundrect_rratio 0.25) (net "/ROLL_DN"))
  (pad "2" smd roundrect (at 1 0) (size 1.2 1.4) (layers "F.Cu" "F.Mask" "F.Paste") (roundrect_rratio 0.25) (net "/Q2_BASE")))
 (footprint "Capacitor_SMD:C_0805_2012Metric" (layer "F.Cu") (at 141 28)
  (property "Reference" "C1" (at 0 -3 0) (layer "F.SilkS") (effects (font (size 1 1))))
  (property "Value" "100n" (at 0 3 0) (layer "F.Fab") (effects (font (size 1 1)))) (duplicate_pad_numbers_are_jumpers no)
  (pad "1" smd roundrect (at -1 0) (size 1.2 1.4) (layers "F.Cu" "F.Mask" "F.Paste") (roundrect_rratio 0.25) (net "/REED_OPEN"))
  (pad "2" smd roundrect (at 1 0) (size 1.2 1.4) (layers "F.Cu" "F.Mask" "F.Paste") (roundrect_rratio 0.25) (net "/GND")))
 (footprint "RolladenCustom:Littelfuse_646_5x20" (layer "F.Cu") (at 37.5 91.1 90)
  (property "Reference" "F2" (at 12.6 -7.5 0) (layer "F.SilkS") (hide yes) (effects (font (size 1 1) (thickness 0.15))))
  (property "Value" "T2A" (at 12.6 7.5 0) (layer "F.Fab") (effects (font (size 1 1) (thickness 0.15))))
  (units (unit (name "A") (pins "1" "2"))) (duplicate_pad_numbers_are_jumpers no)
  (pad "1" thru_hole rect (at 0 0) (size 2.4 2.4) (drill 1.4) (layers "*.Cu" "*.Mask") (remove_unused_layers no) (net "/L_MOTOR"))
  (pad "2" thru_hole circle (at 25.2 0) (size 2.4 2.4) (drill 1.4) (layers "*.Cu" "*.Mask") (remove_unused_layers no) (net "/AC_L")))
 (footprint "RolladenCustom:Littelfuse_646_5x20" (layer "F.Cu") (at 41 27)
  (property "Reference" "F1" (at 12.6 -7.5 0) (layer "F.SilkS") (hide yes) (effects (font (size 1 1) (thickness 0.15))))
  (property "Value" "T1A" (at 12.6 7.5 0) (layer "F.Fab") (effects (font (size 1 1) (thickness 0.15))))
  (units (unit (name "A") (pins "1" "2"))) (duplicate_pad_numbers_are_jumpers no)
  (pad "1" thru_hole rect (at 0 0) (size 2.4 2.4) (drill 1.4) (layers "*.Cu" "*.Mask") (remove_unused_layers no) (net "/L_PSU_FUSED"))
  (pad "2" thru_hole circle (at 25.2 0) (size 2.4 2.4) (drill 1.4) (layers "*.Cu" "*.Mask") (remove_unused_layers no) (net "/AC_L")))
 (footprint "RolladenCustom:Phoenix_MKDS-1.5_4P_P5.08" (layer "F.Cu") (at 104 90)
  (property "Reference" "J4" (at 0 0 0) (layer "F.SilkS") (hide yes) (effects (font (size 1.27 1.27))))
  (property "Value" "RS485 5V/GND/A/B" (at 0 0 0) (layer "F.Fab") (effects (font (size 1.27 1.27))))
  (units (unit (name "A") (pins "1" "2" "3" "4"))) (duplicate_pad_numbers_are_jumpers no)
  (pad "1" thru_hole rect (at 0 0) (size 2.4 2.4) (drill 1.2) (layers "*.Cu" "*.Mask") (remove_unused_layers no) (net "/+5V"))
  (pad "2" thru_hole circle (at 5.08 0) (size 2.4 2.4) (drill 1.2) (layers "*.Cu" "*.Mask") (remove_unused_layers no) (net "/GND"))
  (pad "3" thru_hole circle (at 10.16 0) (size 2.4 2.4) (drill 1.2) (layers "*.Cu" "*.Mask") (remove_unused_layers no) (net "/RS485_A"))
  (pad "4" thru_hole circle (at 15.24 0) (size 2.4 2.4) (drill 1.2) (layers "*.Cu" "*.Mask") (remove_unused_layers no) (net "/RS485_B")))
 (gr_rect (start 20 20) (end 170 110) (stroke (width 0.5) (type default)) (fill no) (layer "Edge.Cuts"))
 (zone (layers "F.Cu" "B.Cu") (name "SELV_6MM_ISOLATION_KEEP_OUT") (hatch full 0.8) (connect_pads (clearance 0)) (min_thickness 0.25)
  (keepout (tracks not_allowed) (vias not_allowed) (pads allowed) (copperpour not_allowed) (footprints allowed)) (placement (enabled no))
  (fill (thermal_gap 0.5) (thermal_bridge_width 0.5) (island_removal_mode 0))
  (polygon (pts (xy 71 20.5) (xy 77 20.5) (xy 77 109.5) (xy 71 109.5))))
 (segment (start 33.16 25) (end 36 25) (width 2) (layer "F.Cu") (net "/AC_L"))
 (segment (start 36 25) (end 36 22.5) (width 2) (layer "F.Cu") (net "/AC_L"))
 (segment (start 36 22.5) (end 66.2 22.5) (width 2) (layer "F.Cu") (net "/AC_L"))
 (segment (start 66.2 22.5) (end 66.2 27) (width 2) (layer "F.Cu") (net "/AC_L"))
 (segment (start 66.2 27) (end 68 27) (width 2) (layer "B.Cu") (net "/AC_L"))
 (segment (start 68 27) (end 68 65.9) (width 2) (layer "B.Cu") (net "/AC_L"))
 (segment (start 68 65.9) (end 37.5 65.9) (width 2) (layer "B.Cu") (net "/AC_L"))
 (segment (start 41 27) (end 41 31) (width 2) (layer "F.Cu") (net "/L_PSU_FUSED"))
 (segment (start 41 31) (end 59.5 31) (width 2) (layer "F.Cu") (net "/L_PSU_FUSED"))
 (segment (start 59.5 31) (end 59.5 27) (width 2) (layer "F.Cu") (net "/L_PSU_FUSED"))
 (segment (start 41 31) (end 32.5 31) (width 2) (layer "F.Cu") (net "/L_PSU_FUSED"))
 (segment (start 32.5 31) (end 32.5 58.3) (width 2) (layer "F.Cu") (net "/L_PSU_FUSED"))
 (segment (start 32.5 58.3) (end 35 58.3) (width 2) (layer "F.Cu") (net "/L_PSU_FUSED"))
 (segment (start 28.08 25) (end 28.08 34) (width 2) (layer "B.Cu") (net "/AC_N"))
 (segment (start 28.08 34) (end 35 34) (width 2) (layer "B.Cu") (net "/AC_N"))
 (segment (start 35 34) (end 35 38) (width 2) (layer "B.Cu") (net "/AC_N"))
 (segment (start 35 34) (end 52 34) (width 2) (layer "B.Cu") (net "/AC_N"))
 (segment (start 52 34) (end 52 27) (width 2) (layer "B.Cu") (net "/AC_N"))
 (segment (start 28.08 34) (end 24.5 34) (width 2) (layer "B.Cu") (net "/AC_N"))
 (segment (start 24.5 34) (end 24.5 102) (width 2) (layer "B.Cu") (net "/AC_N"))
 (segment (start 24.5 102) (end 53 102) (width 2) (layer "B.Cu") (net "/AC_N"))
 (segment (start 23 25) (end 23 106) (width 2) (layer "F.Cu") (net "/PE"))
 (segment (start 23 106) (end 58.08 106) (width 2) (layer "F.Cu") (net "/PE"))
 (segment (start 58.08 106) (end 58.08 102) (width 2) (layer "F.Cu") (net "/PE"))
 (segment (start 37.5 91.1) (end 52 91.1) (width 2) (layer "B.Cu") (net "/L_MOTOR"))
 (segment (start 52 91.1) (end 52 82) (width 2) (layer "B.Cu") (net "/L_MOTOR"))
 (segment (start 52 82) (end 60.18 82) (width 2) (layer "B.Cu") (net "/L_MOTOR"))
 (segment (start 60.18 82) (end 60.18 85.5) (width 2) (layer "B.Cu") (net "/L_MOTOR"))
 (segment (start 52 82) (end 52 72) (width 2) (layer "B.Cu") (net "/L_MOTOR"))
 (segment (start 52 72) (end 60.18 72) (width 2) (layer "B.Cu") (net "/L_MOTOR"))
 (segment (start 60.18 72) (end 60.18 69) (width 2) (layer "B.Cu") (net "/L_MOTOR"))
 (segment (start 60.18 76.62) (end 60.18 79.5) (width 2) (layer "F.Cu") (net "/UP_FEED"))
 (segment (start 60.18 79.5) (end 68.5 79.5) (width 2) (layer "F.Cu") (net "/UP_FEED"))
 (segment (start 68.5 79.5) (end 68.5 82.5) (width 2) (layer "F.Cu") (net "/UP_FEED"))
 (segment (start 68.5 82.5) (end 65.18 82.5) (width 2) (layer "F.Cu") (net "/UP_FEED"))
 (segment (start 65.18 82.5) (end 65.18 85.5) (width 2) (layer "F.Cu") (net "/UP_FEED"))
 (segment (start 65.18 69) (end 68.5 69) (width 2) (layer "B.Cu") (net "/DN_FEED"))
 (segment (start 68.5 69) (end 68.5 90) (width 2) (layer "B.Cu") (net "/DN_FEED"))
 (segment (start 68.5 90) (end 60.18 90) (width 2) (layer "B.Cu") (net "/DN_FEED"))
 (segment (start 60.18 90) (end 60.18 93.12) (width 2) (layer "B.Cu") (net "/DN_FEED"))
 (segment (start 55.18 76.62) (end 55.18 80) (width 2) (layer "F.Cu") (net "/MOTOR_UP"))
 (segment (start 55.18 80) (end 45 80) (width 2) (layer "F.Cu") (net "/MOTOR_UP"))
 (segment (start 45 80) (end 45 97) (width 2) (layer "F.Cu") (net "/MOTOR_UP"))
 (segment (start 45 97) (end 63.16 97) (width 2) (layer "F.Cu") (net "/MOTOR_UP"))
 (segment (start 63.16 97) (end 63.16 102) (width 2) (layer "F.Cu") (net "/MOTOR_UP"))
 (segment (start 55.18 93.12) (end 55.18 98.5) (width 2) (layer "B.Cu") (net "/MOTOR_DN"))
 (segment (start 55.18 98.5) (end 68.24 98.5) (width 2) (layer "B.Cu") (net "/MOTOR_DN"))
 (segment (start 68.24 98.5) (end 68.24 102) (width 2) (layer "B.Cu") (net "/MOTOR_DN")))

